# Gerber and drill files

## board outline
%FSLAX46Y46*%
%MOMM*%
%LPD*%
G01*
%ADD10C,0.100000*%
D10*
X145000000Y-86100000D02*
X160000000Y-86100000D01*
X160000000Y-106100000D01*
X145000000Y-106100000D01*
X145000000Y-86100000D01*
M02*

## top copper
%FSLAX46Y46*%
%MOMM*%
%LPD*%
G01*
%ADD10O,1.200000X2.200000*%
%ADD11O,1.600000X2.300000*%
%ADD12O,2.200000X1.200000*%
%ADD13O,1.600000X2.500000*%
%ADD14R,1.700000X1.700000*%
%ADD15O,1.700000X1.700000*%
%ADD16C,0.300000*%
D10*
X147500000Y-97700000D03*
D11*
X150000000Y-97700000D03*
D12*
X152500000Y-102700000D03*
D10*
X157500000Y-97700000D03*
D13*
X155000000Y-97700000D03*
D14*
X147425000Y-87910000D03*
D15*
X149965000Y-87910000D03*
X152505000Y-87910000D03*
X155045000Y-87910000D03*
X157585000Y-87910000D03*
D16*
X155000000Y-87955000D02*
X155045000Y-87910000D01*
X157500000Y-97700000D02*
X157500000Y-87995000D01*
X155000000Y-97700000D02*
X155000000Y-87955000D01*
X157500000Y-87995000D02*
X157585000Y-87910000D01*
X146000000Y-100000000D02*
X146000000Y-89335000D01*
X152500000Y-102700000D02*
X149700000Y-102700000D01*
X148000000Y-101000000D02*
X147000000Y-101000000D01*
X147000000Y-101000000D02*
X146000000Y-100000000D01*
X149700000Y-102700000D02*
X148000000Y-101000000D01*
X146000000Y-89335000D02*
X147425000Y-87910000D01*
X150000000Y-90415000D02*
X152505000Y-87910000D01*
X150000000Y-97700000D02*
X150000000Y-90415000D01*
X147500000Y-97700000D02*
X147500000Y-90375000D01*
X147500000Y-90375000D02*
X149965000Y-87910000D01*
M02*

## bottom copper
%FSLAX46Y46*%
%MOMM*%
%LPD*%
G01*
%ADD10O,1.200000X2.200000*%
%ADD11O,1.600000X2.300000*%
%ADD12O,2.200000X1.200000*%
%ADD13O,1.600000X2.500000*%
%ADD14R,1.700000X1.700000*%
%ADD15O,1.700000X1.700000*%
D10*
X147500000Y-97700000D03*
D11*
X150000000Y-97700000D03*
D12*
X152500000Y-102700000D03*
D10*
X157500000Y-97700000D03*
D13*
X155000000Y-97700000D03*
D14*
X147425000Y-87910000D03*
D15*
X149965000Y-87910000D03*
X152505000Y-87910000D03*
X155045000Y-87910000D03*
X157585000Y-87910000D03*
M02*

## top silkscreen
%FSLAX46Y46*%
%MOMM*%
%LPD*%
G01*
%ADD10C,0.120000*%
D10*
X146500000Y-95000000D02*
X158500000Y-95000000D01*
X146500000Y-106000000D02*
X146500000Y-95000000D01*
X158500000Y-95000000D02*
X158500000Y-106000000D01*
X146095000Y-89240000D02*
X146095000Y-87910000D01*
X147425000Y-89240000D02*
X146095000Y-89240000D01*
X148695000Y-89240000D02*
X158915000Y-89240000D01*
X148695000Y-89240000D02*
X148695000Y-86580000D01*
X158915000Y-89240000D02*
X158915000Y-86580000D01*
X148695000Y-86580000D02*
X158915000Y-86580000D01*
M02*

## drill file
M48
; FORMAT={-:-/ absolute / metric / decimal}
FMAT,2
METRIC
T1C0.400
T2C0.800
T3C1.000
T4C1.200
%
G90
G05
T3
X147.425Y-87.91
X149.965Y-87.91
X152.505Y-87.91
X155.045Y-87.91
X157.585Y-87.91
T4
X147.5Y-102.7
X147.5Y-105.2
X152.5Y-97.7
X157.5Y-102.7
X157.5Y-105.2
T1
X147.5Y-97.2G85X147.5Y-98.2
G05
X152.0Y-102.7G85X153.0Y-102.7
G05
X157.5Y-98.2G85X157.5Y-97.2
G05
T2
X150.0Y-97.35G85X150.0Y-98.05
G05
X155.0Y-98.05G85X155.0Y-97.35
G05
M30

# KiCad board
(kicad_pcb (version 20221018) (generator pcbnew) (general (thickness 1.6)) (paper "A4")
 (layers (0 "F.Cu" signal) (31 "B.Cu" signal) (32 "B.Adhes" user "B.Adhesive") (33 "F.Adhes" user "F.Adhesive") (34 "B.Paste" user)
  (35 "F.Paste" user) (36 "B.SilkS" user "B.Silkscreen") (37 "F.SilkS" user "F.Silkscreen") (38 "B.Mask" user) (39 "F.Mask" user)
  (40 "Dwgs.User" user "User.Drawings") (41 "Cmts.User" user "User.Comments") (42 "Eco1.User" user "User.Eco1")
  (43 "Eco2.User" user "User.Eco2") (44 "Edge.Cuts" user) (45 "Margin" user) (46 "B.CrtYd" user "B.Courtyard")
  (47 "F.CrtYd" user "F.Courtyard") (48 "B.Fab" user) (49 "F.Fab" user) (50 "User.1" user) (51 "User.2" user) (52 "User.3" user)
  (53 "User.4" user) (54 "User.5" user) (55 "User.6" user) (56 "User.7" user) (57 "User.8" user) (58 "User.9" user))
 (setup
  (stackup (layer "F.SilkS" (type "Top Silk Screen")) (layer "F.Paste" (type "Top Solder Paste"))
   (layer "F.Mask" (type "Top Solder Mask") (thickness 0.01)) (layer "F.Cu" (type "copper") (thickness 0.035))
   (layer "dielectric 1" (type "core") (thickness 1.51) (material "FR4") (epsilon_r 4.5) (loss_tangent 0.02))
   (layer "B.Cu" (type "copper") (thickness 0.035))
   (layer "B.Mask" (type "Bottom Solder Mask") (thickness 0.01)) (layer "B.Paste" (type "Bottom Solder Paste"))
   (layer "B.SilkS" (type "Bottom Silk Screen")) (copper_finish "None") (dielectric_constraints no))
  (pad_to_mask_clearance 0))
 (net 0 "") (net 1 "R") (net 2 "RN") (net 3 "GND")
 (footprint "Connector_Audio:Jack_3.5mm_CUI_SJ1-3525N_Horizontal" (layer "F.Cu") (at 152.5 102.7)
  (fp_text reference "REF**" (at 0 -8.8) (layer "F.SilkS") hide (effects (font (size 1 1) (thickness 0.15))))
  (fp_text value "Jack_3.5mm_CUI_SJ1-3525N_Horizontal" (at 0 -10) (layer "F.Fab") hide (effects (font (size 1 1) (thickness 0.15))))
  (fp_line (start -6 -7.7) (end 6 -7.7) (stroke (width 0.12) (type solid)) (layer "F.SilkS"))
  (fp_line (start -6 3.3) (end -6 -7.7) (stroke (width 0.12) (type solid)) (layer "F.SilkS"))
  (fp_line (start 6 -7.7) (end 6 3.3) (stroke (width 0.12) (type solid)) (layer "F.SilkS"))
  (pad "" np_thru_hole circle (at -5 0) (size 1.2 1.2) (drill 1.2) (layers "F&B.Cu" "*.Mask"))
  (pad "" np_thru_hole circle (at -5 2.5) (size 1.2 1.2) (drill 1.2) (layers "F&B.Cu" "*.Mask"))
  (pad "" np_thru_hole circle (at 0 -5) (size 1.2 1.2) (drill 1.2) (layers "F&B.Cu" "*.Mask"))
  (pad "" np_thru_hole circle (at 5 0) (size 1.2 1.2) (drill 1.2) (layers "F&B.Cu" "*.Mask"))
  (pad "" np_thru_hole circle (at 5 2.5) (size 1.2 1.2) (drill 1.2) (layers "F&B.Cu" "*.Mask"))
  (pad "R" thru_hole oval (at -5 -5) (size 1.2 2.2) (drill oval 0.4 1.4) (layers "*.Cu" "*.Mask") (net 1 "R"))
  (pad "RN" thru_hole oval (at -2.5 -5) (size 1.6 2.3) (drill oval 0.8 1.5) (layers "*.Cu" "*.Mask") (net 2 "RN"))
  (pad "S" thru_hole oval (at 0 0) (size 2.2 1.2) (drill oval 1.4 0.4) (layers "*.Cu" "*.Mask") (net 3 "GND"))
  (pad "T" thru_hole oval (at 5 -5 180) (size 1.2 2.2) (drill oval 0.4 1.4) (layers "*.Cu" "*.Mask"))
  (pad "TN" thru_hole oval (at 2.5 -5 180) (size 1.6 2.5) (drill oval 0.8 1.5) (layers "*.Cu" "*.Mask")))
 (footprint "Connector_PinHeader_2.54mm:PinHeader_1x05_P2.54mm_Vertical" (layer "F.Cu") (at 147.425 87.91 90)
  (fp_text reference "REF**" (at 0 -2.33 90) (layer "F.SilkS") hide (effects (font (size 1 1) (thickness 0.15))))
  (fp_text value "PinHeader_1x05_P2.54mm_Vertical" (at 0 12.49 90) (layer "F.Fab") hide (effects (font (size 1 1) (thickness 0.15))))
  (fp_line (start -1.33 -1.33) (end 0 -1.33) (stroke (width 0.12) (type solid)) (layer "F.SilkS"))
  (fp_line (start -1.33 0) (end -1.33 -1.33) (stroke (width 0.12) (type solid)) (layer "F.SilkS"))
  (fp_line (start -1.33 1.27) (end -1.33 11.49) (stroke (width 0.12) (type solid)) (layer "F.SilkS"))
  (fp_line (start -1.33 1.27) (end 1.33 1.27) (stroke (width 0.12) (type solid)) (layer "F.SilkS"))
  (fp_line (start -1.33 11.49) (end 1.33 11.49) (stroke (width 0.12) (type solid)) (layer "F.SilkS"))
  (fp_line (start 1.33 1.27) (end 1.33 11.49) (stroke (width 0.12) (type solid)) (layer "F.SilkS"))
  (pad "1" thru_hole rect (at 0 0 90) (size 1.7 1.7) (drill 1) (layers "*.Cu" "*.Mask") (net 3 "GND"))
  (pad "2" thru_hole oval (at 0 2.54 90) (size 1.7 1.7) (drill 1) (layers "*.Cu" "*.Mask") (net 1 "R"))
  (pad "3" thru_hole oval (at 0 5.08 90) (size 1.7 1.7) (drill 1) (layers "*.Cu" "*.Mask") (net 2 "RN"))
  (pad "4" thru_hole oval (at 0 7.62 90) (size 1.7 1.7) (drill 1) (layers "*.Cu" "*.Mask"))
  (pad "5" thru_hole oval (at 0 10.16 90) (size 1.7 1.7) (drill 1) (layers "*.Cu" "*.Mask")))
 (gr_rect (start 145 86.1) (end 160 106.1) (stroke (width 0.1) (type default)) (fill none) (layer "Edge.Cuts"))
 (segment (start 155 87.955) (end 155.045 87.91) (width 0.3) (layer "F.Cu") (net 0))
 (segment (start 157.5 97.7) (end 157.5 87.995) (width 0.3) (layer "F.Cu") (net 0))
 (segment (start 155 97.7) (end 155 87.955) (width 0.3) (layer "F.Cu") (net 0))
 (segment (start 157.5 87.995) (end 157.585 87.91) (width 0.3) (layer "F.Cu") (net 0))
 (segment (start 146 100) (end 146 89.335) (width 0.3) (layer "F.Cu") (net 3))
 (segment (start 152.5 102.7) (end 149.7 102.7) (width 0.3) (layer "F.Cu") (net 3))
 (segment (start 148 101) (end 147 101) (width 0.3) (layer "F.Cu") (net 3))
 (segment (start 147 101) (end 146 100) (width 0.3) (layer "F.Cu") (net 3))
 (segment (start 149.7 102.7) (end 148 101) (width 0.3) (layer "F.Cu") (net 3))
 (segment (start 146 89.335) (end 147.425 87.91) (width 0.3) (layer "F.Cu") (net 3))
 (segment (start 150 90.415) (end 152.505 87.91) (width 0.3) (layer "F.Cu") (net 2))
 (segment (start 150 97.7) (end 150 90.415) (width 0.3) (layer "F.Cu") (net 2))
 (segment (start 147.5 97.7) (end 147.5 90.375) (width 0.3) (layer "F.Cu") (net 1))
 (segment (start 147.5 90.375) (end 149.965 87.91) (width 0.3) (layer "F.Cu") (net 1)))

